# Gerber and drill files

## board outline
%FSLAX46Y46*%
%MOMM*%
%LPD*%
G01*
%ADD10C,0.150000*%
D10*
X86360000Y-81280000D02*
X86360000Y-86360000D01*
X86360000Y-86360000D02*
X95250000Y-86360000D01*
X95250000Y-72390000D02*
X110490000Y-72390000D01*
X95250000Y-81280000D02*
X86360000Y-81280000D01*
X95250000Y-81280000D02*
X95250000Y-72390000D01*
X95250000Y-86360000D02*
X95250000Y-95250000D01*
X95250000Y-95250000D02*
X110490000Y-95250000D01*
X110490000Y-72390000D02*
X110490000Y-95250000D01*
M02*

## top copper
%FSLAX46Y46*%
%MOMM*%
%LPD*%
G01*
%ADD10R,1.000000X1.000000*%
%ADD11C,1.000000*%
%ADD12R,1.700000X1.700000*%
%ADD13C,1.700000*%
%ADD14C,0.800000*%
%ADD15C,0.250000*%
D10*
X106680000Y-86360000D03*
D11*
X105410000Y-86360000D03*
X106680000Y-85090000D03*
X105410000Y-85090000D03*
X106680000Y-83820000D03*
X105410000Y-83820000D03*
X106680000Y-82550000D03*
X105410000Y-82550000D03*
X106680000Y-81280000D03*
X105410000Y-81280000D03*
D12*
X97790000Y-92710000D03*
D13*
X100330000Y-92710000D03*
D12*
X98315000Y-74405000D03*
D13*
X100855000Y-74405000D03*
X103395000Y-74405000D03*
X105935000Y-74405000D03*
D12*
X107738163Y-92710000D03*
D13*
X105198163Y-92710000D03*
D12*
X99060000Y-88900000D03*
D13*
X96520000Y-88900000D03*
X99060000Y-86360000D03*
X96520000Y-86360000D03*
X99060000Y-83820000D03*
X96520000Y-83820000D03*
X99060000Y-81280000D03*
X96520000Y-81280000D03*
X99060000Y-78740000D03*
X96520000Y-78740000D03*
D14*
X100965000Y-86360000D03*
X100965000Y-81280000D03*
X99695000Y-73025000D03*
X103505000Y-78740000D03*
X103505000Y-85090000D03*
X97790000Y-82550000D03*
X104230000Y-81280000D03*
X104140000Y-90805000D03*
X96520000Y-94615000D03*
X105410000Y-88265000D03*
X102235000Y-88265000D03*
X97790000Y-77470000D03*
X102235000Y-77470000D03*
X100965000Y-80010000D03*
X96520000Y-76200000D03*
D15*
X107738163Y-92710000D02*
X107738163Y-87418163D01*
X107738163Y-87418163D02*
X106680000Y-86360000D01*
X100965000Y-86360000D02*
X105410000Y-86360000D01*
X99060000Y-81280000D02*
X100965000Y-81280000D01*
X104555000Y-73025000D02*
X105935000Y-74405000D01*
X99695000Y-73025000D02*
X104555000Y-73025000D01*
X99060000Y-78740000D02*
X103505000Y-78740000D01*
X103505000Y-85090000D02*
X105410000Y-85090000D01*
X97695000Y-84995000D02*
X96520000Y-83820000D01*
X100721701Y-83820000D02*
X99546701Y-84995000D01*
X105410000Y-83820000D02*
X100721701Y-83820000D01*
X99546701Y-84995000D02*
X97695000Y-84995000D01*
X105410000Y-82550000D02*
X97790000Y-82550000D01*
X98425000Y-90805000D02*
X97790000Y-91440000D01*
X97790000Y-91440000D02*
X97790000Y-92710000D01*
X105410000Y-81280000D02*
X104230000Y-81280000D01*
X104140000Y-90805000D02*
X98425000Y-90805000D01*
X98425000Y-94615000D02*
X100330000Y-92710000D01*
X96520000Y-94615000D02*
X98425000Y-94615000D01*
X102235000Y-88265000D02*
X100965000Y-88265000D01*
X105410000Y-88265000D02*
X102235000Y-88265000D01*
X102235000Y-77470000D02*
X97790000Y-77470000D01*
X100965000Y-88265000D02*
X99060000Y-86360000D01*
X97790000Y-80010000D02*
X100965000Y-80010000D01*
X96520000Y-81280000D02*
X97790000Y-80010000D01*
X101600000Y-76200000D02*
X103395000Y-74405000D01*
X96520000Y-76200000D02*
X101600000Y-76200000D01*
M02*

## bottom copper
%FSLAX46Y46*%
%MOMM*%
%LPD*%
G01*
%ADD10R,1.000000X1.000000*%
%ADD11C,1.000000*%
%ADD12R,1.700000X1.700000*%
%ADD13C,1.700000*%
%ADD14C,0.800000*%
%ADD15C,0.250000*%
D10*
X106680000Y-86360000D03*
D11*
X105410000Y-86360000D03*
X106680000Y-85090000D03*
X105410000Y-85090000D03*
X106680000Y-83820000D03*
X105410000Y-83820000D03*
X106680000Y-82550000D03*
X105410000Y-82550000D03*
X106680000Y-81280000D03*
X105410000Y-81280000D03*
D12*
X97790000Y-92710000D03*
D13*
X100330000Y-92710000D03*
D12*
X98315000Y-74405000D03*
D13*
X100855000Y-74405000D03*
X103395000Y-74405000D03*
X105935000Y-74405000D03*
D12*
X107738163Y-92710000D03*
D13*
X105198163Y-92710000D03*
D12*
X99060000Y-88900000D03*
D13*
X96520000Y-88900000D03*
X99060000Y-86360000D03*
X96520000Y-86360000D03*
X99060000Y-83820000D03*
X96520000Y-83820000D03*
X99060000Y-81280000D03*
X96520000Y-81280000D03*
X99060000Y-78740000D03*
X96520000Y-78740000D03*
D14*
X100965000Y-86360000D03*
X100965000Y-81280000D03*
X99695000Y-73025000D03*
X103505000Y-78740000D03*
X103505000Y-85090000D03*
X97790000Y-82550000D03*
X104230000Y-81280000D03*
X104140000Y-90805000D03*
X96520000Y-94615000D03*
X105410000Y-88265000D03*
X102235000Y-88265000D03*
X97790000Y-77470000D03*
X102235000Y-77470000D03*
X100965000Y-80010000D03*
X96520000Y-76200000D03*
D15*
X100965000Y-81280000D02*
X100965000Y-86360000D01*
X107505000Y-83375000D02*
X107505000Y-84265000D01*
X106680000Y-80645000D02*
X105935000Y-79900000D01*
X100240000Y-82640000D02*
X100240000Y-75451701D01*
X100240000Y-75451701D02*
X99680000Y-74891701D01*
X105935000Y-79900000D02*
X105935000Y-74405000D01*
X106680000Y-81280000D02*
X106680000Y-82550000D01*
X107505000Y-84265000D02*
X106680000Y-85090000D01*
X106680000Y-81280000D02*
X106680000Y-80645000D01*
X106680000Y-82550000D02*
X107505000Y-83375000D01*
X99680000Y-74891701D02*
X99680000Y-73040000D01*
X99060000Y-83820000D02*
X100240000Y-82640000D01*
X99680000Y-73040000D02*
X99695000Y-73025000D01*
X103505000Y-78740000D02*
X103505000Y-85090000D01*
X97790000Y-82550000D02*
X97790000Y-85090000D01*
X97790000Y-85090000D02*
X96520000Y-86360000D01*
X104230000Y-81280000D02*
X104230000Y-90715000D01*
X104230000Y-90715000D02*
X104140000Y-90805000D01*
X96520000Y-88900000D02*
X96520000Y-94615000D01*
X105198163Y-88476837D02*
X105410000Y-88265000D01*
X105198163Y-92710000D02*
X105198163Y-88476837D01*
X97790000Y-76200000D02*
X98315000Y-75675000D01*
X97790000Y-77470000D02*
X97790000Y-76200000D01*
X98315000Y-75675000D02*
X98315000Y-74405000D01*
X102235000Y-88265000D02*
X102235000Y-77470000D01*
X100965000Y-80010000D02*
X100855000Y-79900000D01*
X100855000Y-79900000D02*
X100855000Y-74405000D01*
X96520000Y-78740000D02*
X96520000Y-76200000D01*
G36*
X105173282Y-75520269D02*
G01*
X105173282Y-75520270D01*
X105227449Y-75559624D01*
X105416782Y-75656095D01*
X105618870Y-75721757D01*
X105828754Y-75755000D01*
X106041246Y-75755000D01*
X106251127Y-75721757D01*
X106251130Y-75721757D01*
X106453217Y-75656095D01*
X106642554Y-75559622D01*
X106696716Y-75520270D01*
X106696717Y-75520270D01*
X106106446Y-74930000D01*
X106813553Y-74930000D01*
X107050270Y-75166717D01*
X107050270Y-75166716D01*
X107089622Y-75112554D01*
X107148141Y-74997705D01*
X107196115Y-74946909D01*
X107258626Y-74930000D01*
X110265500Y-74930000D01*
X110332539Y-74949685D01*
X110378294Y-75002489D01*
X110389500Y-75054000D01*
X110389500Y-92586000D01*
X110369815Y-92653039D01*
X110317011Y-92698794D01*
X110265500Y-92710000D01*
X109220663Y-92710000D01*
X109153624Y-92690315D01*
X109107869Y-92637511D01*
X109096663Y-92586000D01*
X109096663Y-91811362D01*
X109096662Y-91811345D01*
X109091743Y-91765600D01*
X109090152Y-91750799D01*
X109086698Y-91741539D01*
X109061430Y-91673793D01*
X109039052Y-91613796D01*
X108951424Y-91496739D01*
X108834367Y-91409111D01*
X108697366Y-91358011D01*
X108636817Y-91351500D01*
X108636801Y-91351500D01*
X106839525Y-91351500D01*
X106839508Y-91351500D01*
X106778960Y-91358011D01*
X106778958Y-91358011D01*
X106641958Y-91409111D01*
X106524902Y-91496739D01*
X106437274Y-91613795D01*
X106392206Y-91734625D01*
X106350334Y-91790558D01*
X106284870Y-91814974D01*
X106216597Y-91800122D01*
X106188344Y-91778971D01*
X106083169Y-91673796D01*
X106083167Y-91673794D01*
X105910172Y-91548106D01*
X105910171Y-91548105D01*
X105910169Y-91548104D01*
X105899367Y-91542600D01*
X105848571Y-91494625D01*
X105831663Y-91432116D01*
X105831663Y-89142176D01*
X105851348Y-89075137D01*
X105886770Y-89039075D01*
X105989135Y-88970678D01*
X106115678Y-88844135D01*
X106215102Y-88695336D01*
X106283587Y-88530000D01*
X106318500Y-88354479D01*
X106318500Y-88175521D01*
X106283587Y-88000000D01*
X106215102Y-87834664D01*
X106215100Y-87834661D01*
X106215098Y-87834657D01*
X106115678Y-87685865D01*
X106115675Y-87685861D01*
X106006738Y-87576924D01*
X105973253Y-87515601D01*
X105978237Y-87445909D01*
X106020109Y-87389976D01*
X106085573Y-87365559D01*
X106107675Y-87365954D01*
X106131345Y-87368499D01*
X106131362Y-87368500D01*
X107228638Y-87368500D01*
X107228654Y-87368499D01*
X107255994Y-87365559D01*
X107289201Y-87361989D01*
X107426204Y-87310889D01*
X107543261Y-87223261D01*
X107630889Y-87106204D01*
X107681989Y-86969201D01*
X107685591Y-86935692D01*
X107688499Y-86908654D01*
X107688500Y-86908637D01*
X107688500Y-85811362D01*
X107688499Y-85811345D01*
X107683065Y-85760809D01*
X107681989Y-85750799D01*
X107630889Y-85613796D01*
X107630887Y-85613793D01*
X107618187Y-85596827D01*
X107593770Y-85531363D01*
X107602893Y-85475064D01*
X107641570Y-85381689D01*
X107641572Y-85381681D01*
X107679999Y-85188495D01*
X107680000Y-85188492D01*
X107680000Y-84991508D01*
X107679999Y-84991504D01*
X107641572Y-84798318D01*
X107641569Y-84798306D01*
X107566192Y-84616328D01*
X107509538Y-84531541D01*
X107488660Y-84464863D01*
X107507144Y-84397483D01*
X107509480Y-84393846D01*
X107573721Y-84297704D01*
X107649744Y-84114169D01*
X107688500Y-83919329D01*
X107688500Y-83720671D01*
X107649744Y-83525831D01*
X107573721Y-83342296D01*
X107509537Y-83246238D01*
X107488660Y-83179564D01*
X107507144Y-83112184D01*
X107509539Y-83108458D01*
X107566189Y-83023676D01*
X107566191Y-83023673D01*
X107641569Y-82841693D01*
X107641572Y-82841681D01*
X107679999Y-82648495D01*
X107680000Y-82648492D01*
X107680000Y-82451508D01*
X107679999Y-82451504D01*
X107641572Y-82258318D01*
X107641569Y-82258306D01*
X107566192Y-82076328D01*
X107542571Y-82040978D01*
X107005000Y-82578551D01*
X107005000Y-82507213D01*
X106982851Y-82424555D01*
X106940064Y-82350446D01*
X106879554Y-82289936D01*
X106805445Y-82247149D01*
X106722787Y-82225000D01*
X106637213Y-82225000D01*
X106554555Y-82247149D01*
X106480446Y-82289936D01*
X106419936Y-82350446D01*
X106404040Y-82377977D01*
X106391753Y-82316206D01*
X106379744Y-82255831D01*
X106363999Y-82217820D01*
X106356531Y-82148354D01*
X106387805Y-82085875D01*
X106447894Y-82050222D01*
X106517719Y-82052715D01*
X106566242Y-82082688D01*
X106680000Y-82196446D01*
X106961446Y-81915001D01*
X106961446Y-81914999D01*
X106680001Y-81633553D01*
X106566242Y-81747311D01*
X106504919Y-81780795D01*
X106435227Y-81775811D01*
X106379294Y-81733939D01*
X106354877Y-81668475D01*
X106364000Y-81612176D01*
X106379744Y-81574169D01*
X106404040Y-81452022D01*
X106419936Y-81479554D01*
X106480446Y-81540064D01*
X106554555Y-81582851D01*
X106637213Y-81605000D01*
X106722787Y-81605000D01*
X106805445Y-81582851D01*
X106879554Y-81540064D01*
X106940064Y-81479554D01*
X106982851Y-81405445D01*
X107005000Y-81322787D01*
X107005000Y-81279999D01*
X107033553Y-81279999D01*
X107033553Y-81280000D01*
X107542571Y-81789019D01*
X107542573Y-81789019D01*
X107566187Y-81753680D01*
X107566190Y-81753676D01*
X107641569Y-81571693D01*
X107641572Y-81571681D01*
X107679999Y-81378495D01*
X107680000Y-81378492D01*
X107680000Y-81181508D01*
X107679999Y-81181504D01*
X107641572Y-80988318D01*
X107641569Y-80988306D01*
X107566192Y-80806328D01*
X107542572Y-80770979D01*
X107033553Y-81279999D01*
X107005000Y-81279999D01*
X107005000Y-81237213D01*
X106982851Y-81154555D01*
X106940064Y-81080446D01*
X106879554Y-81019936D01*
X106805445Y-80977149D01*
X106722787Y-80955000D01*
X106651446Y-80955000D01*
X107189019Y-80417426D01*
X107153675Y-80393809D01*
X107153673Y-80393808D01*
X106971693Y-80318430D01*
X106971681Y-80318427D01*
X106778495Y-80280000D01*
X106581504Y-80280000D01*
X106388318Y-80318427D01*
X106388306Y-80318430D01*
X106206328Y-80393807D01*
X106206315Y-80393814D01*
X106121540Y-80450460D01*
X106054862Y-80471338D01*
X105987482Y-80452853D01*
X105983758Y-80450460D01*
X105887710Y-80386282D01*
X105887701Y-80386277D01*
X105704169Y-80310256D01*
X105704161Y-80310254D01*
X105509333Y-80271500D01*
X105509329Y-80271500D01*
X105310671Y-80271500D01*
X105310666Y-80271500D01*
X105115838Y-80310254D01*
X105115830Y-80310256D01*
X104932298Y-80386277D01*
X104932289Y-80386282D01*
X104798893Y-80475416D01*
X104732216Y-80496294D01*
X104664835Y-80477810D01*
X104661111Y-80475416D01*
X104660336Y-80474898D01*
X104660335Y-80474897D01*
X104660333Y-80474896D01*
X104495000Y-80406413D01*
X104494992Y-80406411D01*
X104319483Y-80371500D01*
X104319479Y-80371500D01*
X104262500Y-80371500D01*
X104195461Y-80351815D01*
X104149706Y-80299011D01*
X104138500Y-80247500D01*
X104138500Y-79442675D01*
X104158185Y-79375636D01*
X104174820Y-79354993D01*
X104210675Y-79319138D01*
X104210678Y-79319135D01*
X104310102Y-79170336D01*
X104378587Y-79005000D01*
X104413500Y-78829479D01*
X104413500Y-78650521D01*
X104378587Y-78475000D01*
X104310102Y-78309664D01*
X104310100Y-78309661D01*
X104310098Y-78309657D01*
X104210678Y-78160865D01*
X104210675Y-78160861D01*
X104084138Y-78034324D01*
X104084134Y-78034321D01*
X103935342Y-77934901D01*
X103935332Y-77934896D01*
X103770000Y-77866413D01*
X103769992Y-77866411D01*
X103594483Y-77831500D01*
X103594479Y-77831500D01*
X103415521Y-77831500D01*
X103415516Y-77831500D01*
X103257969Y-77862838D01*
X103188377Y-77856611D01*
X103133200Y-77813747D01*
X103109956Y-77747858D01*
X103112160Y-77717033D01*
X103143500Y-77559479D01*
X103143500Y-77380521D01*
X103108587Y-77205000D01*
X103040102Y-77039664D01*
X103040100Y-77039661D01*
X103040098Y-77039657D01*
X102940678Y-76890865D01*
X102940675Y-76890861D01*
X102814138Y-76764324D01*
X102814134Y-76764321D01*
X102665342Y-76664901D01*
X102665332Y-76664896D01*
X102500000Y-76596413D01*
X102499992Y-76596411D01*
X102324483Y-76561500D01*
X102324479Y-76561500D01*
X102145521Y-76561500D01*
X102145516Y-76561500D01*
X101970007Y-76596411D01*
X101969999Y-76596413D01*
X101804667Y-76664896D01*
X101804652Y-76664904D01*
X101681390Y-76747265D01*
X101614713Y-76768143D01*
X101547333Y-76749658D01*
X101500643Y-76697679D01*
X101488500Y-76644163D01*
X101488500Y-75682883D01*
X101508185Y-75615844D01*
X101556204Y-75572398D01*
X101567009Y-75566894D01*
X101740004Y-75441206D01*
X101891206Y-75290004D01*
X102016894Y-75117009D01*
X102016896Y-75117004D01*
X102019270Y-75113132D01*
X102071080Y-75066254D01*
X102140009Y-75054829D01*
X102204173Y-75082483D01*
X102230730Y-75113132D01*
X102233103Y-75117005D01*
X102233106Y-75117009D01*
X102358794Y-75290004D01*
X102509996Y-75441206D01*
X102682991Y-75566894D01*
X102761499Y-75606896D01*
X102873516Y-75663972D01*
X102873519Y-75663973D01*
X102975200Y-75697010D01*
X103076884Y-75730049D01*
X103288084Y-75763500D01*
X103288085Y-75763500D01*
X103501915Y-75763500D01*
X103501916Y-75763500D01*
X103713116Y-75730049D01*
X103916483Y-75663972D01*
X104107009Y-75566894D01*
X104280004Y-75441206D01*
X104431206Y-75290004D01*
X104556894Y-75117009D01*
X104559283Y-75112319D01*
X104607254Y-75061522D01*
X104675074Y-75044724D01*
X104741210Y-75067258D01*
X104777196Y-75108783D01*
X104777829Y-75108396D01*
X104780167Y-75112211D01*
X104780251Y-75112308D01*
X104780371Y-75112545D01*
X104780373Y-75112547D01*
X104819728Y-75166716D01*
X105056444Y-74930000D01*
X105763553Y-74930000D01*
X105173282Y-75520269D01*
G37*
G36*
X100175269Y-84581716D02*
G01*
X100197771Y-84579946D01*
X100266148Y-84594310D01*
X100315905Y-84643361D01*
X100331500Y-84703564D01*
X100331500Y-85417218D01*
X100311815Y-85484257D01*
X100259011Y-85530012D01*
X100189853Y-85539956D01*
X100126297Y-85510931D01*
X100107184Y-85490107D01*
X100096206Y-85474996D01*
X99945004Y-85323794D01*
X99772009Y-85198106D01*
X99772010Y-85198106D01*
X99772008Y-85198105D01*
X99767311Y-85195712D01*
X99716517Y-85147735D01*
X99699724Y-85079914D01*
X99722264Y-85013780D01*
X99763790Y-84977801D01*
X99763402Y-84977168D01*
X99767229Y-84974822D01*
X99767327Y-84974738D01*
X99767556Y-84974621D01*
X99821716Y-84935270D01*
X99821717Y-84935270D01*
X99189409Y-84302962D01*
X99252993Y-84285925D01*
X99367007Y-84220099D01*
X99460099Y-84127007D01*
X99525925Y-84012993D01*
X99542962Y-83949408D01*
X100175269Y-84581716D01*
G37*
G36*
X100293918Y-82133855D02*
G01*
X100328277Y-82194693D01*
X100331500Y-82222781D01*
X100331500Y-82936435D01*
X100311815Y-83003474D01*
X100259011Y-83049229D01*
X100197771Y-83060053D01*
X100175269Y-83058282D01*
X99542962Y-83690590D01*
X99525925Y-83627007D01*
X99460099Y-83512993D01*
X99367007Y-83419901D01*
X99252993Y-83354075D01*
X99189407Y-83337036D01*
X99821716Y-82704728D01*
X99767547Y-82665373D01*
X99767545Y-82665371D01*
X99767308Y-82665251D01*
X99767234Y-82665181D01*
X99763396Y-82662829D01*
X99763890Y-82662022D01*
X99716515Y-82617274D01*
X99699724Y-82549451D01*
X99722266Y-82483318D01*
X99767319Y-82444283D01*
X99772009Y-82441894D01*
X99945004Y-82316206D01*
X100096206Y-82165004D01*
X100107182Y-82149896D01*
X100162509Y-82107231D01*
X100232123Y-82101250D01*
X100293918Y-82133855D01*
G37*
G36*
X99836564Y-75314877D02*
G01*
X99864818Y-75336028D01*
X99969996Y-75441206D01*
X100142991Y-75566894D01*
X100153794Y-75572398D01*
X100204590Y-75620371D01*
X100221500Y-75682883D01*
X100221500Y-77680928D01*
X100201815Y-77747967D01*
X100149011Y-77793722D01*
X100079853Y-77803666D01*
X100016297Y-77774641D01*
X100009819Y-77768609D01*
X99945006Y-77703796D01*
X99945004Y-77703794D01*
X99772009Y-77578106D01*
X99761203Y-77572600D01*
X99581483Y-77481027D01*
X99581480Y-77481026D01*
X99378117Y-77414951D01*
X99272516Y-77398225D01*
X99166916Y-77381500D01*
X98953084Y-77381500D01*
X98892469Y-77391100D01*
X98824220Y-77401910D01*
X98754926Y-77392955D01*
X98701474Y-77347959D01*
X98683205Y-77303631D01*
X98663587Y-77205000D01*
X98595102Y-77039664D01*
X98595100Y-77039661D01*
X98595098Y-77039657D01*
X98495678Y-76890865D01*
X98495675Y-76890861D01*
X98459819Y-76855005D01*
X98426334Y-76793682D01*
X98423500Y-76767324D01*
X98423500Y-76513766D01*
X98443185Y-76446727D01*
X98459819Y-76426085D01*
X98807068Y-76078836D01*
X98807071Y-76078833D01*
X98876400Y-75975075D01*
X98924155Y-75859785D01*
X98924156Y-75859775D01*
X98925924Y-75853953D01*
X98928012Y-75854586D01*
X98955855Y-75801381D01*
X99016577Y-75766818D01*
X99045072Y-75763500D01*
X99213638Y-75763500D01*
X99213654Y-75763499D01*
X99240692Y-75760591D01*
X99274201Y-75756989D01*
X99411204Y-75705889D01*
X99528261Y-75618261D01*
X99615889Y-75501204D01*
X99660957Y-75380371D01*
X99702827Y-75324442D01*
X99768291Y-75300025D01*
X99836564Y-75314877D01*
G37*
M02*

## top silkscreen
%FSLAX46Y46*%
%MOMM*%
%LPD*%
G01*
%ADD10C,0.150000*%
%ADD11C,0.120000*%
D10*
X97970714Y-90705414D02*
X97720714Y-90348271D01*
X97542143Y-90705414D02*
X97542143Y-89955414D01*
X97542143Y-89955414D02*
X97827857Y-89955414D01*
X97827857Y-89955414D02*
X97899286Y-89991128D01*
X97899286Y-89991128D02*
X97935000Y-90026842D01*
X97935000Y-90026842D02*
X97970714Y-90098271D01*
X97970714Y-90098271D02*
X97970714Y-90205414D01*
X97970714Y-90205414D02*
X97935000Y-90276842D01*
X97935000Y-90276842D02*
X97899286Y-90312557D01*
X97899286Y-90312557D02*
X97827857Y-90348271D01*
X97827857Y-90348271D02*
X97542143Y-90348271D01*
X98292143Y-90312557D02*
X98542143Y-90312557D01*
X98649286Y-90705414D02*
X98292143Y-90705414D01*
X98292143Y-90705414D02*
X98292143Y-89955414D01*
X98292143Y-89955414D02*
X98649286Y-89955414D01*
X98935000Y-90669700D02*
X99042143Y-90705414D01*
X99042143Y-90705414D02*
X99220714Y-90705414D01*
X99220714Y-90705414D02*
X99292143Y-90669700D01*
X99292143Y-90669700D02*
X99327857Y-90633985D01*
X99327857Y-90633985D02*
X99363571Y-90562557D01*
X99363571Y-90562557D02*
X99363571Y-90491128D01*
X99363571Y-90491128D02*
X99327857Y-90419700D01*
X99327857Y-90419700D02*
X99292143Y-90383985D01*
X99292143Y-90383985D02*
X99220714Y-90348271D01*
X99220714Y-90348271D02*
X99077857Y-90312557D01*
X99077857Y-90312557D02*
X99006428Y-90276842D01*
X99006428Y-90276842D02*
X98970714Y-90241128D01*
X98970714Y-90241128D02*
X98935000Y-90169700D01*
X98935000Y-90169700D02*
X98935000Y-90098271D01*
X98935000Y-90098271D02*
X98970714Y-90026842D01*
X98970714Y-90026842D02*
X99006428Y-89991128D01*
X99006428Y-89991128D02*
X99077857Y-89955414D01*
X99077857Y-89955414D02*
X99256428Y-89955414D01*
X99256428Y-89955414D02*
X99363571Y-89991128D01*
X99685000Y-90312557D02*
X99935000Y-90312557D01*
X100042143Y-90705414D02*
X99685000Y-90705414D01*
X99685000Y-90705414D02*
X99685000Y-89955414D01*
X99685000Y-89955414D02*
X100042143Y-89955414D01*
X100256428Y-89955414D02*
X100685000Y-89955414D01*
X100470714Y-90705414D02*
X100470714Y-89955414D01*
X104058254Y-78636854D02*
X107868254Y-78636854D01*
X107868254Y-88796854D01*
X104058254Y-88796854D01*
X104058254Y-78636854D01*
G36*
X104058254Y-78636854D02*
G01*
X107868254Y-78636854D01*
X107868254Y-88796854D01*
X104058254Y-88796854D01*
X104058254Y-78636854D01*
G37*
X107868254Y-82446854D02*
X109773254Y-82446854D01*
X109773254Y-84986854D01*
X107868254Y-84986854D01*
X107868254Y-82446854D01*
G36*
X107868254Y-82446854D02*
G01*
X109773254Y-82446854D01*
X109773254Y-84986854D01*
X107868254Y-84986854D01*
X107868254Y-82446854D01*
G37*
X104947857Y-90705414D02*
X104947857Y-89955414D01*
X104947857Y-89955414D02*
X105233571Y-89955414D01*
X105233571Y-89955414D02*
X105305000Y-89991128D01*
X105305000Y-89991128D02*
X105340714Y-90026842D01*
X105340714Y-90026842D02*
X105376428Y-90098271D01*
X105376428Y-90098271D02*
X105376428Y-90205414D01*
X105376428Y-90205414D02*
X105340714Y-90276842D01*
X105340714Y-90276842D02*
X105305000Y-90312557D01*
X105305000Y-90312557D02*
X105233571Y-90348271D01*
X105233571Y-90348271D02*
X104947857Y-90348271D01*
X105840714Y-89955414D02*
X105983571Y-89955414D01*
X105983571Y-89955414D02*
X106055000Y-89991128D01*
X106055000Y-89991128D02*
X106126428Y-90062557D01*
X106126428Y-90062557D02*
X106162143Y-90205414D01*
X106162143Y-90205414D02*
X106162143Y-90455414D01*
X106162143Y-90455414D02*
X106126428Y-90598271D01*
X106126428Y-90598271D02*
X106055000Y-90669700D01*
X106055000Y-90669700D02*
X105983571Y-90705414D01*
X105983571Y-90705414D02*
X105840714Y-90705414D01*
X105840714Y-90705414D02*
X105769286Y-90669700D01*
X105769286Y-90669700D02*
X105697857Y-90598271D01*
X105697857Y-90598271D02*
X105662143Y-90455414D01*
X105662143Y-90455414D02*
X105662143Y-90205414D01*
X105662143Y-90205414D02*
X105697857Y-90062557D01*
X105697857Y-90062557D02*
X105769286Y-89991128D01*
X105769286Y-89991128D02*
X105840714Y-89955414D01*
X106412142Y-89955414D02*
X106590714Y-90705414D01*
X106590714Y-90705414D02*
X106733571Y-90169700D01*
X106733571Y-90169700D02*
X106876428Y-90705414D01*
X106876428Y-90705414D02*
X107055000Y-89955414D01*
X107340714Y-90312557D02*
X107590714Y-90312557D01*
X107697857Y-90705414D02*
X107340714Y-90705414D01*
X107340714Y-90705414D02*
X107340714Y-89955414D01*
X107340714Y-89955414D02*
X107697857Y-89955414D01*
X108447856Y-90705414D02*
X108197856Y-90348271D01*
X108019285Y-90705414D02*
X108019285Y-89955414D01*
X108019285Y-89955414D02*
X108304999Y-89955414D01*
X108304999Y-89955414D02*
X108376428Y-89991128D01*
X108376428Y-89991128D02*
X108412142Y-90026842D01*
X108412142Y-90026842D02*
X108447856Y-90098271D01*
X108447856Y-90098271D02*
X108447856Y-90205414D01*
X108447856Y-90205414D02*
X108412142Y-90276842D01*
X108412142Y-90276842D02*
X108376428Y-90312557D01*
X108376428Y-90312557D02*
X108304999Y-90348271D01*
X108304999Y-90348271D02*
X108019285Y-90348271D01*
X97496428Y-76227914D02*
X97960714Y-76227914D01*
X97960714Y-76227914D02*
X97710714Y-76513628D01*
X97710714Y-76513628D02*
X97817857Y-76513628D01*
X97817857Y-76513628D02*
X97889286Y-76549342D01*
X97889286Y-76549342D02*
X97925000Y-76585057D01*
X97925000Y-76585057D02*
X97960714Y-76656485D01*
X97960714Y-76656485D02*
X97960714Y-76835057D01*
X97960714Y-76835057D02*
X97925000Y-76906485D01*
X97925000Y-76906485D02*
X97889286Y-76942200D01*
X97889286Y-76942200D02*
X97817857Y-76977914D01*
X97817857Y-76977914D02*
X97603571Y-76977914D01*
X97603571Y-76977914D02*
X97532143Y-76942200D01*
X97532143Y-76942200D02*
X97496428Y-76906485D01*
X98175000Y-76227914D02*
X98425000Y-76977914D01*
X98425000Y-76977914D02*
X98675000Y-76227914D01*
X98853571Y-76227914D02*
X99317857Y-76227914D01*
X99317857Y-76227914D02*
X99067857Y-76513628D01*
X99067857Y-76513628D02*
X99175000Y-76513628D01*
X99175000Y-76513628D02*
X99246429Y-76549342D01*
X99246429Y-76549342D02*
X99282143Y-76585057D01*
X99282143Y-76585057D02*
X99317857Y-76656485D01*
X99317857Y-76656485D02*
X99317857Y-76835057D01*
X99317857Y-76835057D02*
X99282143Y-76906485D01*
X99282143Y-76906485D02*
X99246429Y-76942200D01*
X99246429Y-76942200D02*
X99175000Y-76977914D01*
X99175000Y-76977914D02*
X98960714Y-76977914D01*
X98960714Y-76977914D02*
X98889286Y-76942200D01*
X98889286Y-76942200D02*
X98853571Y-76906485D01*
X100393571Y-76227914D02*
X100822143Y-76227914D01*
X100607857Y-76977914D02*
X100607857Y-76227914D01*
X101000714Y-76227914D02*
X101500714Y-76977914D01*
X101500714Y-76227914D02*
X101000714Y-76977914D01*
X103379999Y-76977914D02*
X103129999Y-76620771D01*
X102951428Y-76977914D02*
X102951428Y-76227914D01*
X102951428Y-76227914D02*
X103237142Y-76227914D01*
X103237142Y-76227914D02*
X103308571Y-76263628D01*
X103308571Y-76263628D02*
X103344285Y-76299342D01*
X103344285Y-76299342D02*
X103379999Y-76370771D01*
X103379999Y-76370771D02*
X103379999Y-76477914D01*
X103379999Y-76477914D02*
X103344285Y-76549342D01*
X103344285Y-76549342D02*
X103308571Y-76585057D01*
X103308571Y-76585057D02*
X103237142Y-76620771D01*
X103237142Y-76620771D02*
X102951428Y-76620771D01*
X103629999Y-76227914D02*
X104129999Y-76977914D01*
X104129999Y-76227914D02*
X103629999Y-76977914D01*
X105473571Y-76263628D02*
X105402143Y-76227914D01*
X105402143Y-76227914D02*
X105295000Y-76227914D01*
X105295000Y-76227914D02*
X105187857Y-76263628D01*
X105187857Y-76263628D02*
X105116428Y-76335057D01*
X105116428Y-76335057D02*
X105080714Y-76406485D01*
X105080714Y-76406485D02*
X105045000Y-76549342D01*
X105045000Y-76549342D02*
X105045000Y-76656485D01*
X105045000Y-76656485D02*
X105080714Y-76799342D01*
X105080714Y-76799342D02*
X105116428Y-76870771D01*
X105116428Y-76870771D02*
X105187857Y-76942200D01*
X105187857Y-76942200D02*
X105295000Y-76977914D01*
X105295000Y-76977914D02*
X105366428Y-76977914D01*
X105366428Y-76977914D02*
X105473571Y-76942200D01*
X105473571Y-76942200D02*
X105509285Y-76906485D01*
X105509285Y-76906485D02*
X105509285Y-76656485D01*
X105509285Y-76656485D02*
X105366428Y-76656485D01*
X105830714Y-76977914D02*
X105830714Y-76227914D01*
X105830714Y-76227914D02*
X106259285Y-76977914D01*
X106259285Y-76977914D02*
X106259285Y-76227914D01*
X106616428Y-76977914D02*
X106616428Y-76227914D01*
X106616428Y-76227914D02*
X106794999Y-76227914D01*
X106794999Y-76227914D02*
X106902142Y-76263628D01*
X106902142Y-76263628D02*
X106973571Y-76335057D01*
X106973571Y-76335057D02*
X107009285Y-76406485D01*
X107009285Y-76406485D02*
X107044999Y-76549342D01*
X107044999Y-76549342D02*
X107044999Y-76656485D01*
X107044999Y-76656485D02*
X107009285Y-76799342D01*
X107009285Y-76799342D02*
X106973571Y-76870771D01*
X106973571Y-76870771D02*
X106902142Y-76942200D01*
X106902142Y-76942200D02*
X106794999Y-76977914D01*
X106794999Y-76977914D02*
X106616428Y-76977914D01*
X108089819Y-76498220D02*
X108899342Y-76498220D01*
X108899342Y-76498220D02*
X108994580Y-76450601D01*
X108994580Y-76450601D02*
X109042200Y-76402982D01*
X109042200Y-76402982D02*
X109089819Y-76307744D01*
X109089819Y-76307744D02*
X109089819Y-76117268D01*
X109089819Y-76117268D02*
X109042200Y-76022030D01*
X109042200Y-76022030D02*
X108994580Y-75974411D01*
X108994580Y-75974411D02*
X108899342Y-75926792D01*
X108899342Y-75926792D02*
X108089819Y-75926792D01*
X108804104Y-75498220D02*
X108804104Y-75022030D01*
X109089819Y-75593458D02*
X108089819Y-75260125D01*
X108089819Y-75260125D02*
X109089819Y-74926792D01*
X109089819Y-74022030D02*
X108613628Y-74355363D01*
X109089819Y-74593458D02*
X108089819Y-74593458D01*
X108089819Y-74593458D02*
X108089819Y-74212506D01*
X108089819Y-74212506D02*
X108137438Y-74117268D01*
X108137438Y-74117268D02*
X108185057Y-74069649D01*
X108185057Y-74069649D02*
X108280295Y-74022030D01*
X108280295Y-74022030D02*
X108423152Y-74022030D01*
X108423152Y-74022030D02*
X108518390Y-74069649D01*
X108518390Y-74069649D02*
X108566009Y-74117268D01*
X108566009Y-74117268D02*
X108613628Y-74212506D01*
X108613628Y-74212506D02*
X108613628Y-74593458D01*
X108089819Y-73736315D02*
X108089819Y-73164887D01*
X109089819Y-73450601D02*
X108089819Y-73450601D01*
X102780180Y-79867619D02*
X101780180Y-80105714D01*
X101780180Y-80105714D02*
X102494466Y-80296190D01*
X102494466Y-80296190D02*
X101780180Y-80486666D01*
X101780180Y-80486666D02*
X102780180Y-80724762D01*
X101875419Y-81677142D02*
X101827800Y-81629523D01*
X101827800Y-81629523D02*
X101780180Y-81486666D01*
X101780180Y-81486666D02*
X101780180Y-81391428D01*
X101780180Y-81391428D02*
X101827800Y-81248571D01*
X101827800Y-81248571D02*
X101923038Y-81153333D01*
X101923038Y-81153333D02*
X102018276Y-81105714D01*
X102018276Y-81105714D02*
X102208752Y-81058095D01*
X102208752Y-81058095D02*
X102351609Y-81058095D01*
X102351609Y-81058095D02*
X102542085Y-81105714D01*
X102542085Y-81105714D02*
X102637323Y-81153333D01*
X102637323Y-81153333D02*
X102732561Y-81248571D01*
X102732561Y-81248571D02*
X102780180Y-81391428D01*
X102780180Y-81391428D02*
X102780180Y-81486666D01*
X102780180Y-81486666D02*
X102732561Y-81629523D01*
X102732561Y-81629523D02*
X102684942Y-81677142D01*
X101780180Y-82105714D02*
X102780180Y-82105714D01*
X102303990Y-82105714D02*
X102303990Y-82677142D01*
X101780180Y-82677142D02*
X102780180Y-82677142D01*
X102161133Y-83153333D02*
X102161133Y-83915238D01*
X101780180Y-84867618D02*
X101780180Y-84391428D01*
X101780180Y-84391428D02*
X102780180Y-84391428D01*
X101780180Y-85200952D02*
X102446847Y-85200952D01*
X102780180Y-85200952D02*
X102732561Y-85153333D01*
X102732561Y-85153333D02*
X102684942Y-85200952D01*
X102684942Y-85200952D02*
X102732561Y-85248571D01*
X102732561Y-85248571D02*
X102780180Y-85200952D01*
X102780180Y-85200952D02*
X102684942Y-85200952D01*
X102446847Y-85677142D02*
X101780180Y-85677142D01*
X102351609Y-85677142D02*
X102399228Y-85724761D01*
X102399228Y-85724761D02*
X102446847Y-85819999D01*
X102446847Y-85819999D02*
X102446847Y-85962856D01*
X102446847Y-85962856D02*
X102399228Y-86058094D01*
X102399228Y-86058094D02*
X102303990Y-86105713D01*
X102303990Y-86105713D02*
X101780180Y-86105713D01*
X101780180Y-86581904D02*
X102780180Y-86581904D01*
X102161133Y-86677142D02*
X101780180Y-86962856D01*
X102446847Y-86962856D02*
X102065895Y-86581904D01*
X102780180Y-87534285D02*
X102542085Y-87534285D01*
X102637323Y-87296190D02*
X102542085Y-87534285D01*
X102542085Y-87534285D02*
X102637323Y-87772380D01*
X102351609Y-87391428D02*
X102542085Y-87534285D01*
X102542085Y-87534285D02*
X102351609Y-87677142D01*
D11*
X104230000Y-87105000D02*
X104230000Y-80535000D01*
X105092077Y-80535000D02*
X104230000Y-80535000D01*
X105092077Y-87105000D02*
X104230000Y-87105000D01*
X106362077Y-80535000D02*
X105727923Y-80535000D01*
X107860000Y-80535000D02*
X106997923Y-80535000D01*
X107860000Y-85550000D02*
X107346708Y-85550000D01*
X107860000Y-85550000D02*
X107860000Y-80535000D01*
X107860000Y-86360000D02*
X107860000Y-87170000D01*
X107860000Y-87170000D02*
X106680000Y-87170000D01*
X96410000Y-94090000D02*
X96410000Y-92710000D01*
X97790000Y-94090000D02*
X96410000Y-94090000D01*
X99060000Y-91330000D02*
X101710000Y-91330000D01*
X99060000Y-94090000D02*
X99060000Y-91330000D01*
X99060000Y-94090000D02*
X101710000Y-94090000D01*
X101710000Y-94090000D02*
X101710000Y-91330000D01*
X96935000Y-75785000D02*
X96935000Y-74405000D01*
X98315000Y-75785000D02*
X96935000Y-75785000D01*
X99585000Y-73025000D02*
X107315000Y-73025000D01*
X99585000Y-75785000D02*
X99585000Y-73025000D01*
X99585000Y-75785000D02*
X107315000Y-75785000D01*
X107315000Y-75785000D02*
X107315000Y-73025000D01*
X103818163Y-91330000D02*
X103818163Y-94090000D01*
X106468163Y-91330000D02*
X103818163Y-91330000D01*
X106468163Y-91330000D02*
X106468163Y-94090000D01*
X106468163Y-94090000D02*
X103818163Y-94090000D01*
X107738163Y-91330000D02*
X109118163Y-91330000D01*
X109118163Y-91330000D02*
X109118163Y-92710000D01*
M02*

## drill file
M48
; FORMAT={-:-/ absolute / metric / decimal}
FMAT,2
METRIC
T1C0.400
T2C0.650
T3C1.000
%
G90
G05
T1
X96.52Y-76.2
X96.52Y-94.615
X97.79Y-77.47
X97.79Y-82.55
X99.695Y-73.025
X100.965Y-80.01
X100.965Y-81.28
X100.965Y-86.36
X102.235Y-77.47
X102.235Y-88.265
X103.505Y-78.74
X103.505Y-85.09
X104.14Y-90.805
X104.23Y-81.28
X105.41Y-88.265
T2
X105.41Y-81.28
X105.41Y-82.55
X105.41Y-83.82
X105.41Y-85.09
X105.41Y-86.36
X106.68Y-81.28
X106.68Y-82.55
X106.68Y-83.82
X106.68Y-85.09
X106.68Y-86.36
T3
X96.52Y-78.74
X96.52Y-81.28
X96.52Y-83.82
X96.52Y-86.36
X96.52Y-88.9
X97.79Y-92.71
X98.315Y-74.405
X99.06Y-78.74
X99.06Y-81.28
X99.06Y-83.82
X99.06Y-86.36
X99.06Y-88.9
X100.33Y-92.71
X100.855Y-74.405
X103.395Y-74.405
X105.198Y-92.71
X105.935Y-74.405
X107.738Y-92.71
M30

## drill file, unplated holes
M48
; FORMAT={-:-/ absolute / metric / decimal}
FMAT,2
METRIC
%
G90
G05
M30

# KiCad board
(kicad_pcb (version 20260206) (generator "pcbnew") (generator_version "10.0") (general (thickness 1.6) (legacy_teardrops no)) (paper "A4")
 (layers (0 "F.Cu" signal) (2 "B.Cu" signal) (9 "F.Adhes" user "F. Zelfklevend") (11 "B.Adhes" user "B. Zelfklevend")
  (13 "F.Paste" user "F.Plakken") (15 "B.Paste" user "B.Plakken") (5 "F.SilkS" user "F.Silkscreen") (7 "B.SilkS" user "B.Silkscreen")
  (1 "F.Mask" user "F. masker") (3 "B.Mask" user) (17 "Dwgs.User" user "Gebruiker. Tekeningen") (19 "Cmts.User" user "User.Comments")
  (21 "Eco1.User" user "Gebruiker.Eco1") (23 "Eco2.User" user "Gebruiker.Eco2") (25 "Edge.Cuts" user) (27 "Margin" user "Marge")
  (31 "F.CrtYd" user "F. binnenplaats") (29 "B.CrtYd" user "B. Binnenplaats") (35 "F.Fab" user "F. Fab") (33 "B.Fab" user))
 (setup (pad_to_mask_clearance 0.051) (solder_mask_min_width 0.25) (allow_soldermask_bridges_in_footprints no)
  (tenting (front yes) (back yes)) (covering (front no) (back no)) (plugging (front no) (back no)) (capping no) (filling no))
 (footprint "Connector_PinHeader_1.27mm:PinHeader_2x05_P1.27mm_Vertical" (layer "F.Cu") (at 106.68 86.36 180)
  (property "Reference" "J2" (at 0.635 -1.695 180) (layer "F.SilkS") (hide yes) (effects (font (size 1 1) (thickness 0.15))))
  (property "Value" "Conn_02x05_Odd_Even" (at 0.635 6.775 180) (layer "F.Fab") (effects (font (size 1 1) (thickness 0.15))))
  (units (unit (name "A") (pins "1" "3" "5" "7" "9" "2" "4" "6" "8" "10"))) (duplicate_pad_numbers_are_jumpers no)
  (fp_line (start 2.45 -0.745) (end 2.45 5.825) (stroke (width 0.12) (type solid)) (layer "F.SilkS"))
  (fp_line (start 1.587923 5.825) (end 2.45 5.825) (stroke (width 0.12) (type solid)) (layer "F.SilkS"))
  (fp_line (start 1.587923 -0.745) (end 2.45 -0.745) (stroke (width 0.12) (type solid)) (layer "F.SilkS"))
  (fp_line (start 0.317923 5.825) (end 0.952077 5.825) (stroke (width 0.12) (type solid)) (layer "F.SilkS"))
  (fp_line (start -1.18 5.825) (end -0.317923 5.825) (stroke (width 0.12) (type solid)) (layer "F.SilkS"))
  (fp_line (start -1.18 0.81) (end -0.666708 0.81) (stroke (width 0.12) (type solid)) (layer "F.SilkS"))
  (fp_line (start -1.18 0.81) (end -1.18 5.825) (stroke (width 0.12) (type solid)) (layer "F.SilkS"))
  (fp_line (start -1.18 0) (end -1.18 -0.81) (stroke (width 0.12) (type solid)) (layer "F.SilkS"))
  (fp_line (start -1.18 -0.81) (end 0 -0.81) (stroke (width 0.12) (type solid)) (layer "F.SilkS"))
  (pad "1" thru_hole rect (at 0 0 180) (size 1 1) (drill 0.65) (layers "*.Cu" "*.Mask") (remove_unused_layers no) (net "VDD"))
  (pad "2" thru_hole circle (at 1.27 0 180) (size 1 1) (drill 0.65) (layers "*.Cu" "*.Mask") (remove_unused_layers no) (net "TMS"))
  (pad "3" thru_hole circle (at 0 1.27 180) (size 1 1) (drill 0.65) (layers "*.Cu" "*.Mask") (remove_unused_layers no) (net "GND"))
  (pad "4" thru_hole circle (at 1.27 1.27 180) (size 1 1) (drill 0.65) (layers "*.Cu" "*.Mask") (remove_unused_layers no) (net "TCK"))
  (pad "5" thru_hole circle (at 0 2.54 180) (size 1 1) (drill 0.65) (layers "*.Cu" "*.Mask") (remove_unused_layers no)
   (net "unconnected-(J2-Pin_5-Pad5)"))
  (pad "6" thru_hole circle (at 1.27 2.54 180) (size 1 1) (drill 0.65) (layers "*.Cu" "*.Mask") (remove_unused_layers no) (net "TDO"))
  (pad "7" thru_hole circle (at 0 3.81 180) (size 1 1) (drill 0.65) (layers "*.Cu" "*.Mask") (remove_unused_layers no) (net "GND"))
  (pad "8" thru_hole circle (at 1.27 3.81 180) (size 1 1) (drill 0.65) (layers "*.Cu" "*.Mask") (remove_unused_layers no) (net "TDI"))
  (pad "9" thru_hole circle (at 0 5.08 180) (size 1 1) (drill 0.65) (layers "*.Cu" "*.Mask") (remove_unused_layers no) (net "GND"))
  (pad "10" thru_hole circle (at 1.27 5.08 180) (size 1 1) (drill 0.65) (layers "*.Cu" "*.Mask") (remove_unused_layers no) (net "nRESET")))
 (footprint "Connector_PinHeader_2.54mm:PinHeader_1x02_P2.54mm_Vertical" (layer "F.Cu") (at 97.79 92.71 90)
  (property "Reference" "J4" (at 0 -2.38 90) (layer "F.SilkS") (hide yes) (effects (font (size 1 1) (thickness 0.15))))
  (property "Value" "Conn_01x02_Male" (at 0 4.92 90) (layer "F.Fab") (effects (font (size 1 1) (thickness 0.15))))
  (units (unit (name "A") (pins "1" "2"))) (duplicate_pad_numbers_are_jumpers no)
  (fp_line (start -1.38 -1.38) (end 0 -1.38) (stroke (width 0.12) (type solid)) (layer "F.SilkS"))
  (fp_line (start -1.38 0) (end -1.38 -1.38) (stroke (width 0.12) (type solid)) (layer "F.SilkS"))
  (fp_line (start 1.38 1.27) (end 1.38 3.92) (stroke (width 0.12) (type solid)) (layer "F.SilkS"))
  (fp_line (start -1.38 1.27) (end 1.38 1.27) (stroke (width 0.12) (type solid)) (layer "F.SilkS"))
  (fp_line (start -1.38 1.27) (end -1.38 3.92) (stroke (width 0.12) (type solid)) (layer "F.SilkS"))
  (fp_line (start -1.38 3.92) (end 1.38 3.92) (stroke (width 0.12) (type solid)) (layer "F.SilkS"))
  (pad "1" thru_hole rect (at 0 0 90) (size 1.7 1.7) (drill 1) (layers "*.Cu" "*.Mask") (remove_unused_layers no) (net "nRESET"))
  (pad "2" thru_hole circle (at 0 2.54 90) (size 1.7 1.7) (drill 1) (layers "*.Cu" "*.Mask") (remove_unused_layers no) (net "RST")))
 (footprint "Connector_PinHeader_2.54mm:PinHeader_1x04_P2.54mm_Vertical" (layer "F.Cu") (at 98.315 74.405 90)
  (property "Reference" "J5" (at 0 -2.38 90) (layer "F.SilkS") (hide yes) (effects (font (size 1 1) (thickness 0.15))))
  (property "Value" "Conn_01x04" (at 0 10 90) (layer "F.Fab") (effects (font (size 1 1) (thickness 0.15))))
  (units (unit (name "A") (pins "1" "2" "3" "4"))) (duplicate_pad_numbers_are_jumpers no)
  (fp_line (start -1.38 -1.38) (end 0 -1.38) (stroke (width 0.12) (type solid)) (layer "F.SilkS"))
  (fp_line (start -1.38 0) (end -1.38 -1.38) (stroke (width 0.12) (type solid)) (layer "F.SilkS"))
  (fp_line (start 1.38 1.27) (end 1.38 9) (stroke (width 0.12) (type solid)) (layer "F.SilkS"))
  (fp_line (start -1.38 1.27) (end 1.38 1.27) (stroke (width 0.12) (type solid)) (layer "F.SilkS"))
  (fp_line (start -1.38 1.27) (end -1.38 9) (stroke (width 0.12) (type solid)) (layer "F.SilkS"))
  (fp_line (start -1.38 9) (end 1.38 9) (stroke (width 0.12) (type solid)) (layer "F.SilkS"))
  (pad "1" thru_hole rect (at 0 0 90) (size 1.7 1.7) (drill 1) (layers "*.Cu" "*.Mask") (remove_unused_layers no) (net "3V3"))
  (pad "2" thru_hole circle (at 0 2.54 90) (size 1.7 1.7) (drill 1) (layers "*.Cu" "*.Mask") (remove_unused_layers no) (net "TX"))
  (pad "3" thru_hole circle (at 0 5.08 90) (size 1.7 1.7) (drill 1) (layers "*.Cu" "*.Mask") (remove_unused_layers no) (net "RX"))
  (pad "4" thru_hole circle (at 0 7.62 90) (size 1.7 1.7) (drill 1) (layers "*.Cu" "*.Mask") (remove_unused_layers no) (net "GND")))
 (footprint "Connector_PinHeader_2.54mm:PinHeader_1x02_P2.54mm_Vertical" (layer "F.Cu") (at 107.738163 92.71 -90)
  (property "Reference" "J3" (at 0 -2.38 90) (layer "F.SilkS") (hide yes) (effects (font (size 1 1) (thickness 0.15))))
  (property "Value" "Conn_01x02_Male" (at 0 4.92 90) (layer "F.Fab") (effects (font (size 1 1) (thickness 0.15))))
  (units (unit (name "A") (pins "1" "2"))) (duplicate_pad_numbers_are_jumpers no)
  (fp_line (start -1.38 3.92) (end 1.38 3.92) (stroke (width 0.12) (type solid)) (layer "F.SilkS"))
  (fp_line (start -1.38 1.27) (end -1.38 3.92) (stroke (width 0.12) (type solid)) (layer "F.SilkS"))
  (fp_line (start -1.38 1.27) (end 1.38 1.27) (stroke (width 0.12) (type solid)) (layer "F.SilkS"))
  (fp_line (start 1.38 1.27) (end 1.38 3.92) (stroke (width 0.12) (type solid)) (layer "F.SilkS"))
  (fp_line (start -1.38 0) (end -1.38 -1.38) (stroke (width 0.12) (type solid)) (layer "F.SilkS"))
  (fp_line (start -1.38 -1.38) (end 0 -1.38) (stroke (width 0.12) (type solid)) (layer "F.SilkS"))
  (pad "1" thru_hole rect (at 0 0 270) (size 1.7 1.7) (drill 1) (layers "*.Cu" "*.Mask") (remove_unused_layers no) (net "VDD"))
  (pad "2" thru_hole circle (at 0 2.54 270) (size 1.7 1.7) (drill 1) (layers "*.Cu" "*.Mask") (remove_unused_layers no) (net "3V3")))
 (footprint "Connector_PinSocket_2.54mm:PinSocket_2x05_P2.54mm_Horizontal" (layer "B.Cu") (at 99.06 88.9)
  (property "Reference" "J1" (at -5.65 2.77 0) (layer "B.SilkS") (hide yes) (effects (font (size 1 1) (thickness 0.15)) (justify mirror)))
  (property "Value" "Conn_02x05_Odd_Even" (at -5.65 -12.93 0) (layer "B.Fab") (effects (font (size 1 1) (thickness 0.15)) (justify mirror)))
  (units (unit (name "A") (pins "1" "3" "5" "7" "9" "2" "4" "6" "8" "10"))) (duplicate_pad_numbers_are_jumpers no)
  (pad "1" thru_hole rect (at 0 0) (size 1.7 1.7) (drill 1) (layers "*.Cu" "*.Mask") (remove_unused_layers no) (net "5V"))
  (pad "2" thru_hole circle (at -2.54 0) (size 1.7 1.7) (drill 1) (layers "*.Cu" "*.Mask") (remove_unused_layers no) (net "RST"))
  (pad "3" thru_hole circle (at 0 -2.54) (size 1.7 1.7) (drill 1) (layers "*.Cu" "*.Mask") (remove_unused_layers no) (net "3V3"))
  (pad "4" thru_hole circle (at -2.54 -2.54) (size 1.7 1.7) (drill 1) (layers "*.Cu" "*.Mask") (remove_unused_layers no) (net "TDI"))
  (pad "5" thru_hole circle (at 0 -5.08) (size 1.7 1.7) (drill 1) (layers "*.Cu" "*.Mask") (remove_unused_layers no) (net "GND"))
  (pad "6" thru_hole circle (at -2.54 -5.08) (size 1.7 1.7) (drill 1) (layers "*.Cu" "*.Mask") (remove_unused_layers no) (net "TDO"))
  (pad "7" thru_hole circle (at 0 -7.62) (size 1.7 1.7) (drill 1) (layers "*.Cu" "*.Mask") (remove_unused_layers no) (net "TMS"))
  (pad "8" thru_hole circle (at -2.54 -7.62) (size 1.7 1.7) (drill 1) (layers "*.Cu" "*.Mask") (remove_unused_layers no) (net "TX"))
  (pad "9" thru_hole circle (at 0 -10.16) (size 1.7 1.7) (drill 1) (layers "*.Cu" "*.Mask") (remove_unused_layers no) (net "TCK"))
  (pad "10" thru_hole circle (at -2.54 -10.16) (size 1.7 1.7) (drill 1) (layers "*.Cu" "*.Mask") (remove_unused_layers no) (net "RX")))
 (gr_rect (start 104.058254 78.636854) (end 107.868254 88.796854) (stroke (width 0.15) (type solid)) (fill yes) (layer "F.SilkS"))
 (gr_rect (start 107.868254 82.446854) (end 109.773254 84.986854) (stroke (width 0.15) (type solid)) (fill yes) (layer "F.SilkS"))
 (gr_line (start 86.36 81.28) (end 86.36 86.36) (stroke (width 0.15) (type default)) (layer "Edge.Cuts"))
 (gr_line (start 86.36 86.36) (end 95.25 86.36) (stroke (width 0.15) (type default)) (layer "Edge.Cuts"))
 (gr_line (start 95.25 72.39) (end 110.49 72.39) (stroke (width 0.15) (type default)) (layer "Edge.Cuts"))
 (gr_line (start 95.25 81.28) (end 86.36 81.28) (stroke (width 0.15) (type default)) (layer "Edge.Cuts"))
 (gr_line (start 95.25 81.28) (end 95.25 72.39) (stroke (width 0.15) (type default)) (layer "Edge.Cuts"))
 (gr_line (start 95.25 86.36) (end 95.25 95.25) (stroke (width 0.15) (type default)) (layer "Edge.Cuts"))
 (gr_line (start 95.25 95.25) (end 110.49 95.25) (stroke (width 0.15) (type default)) (layer "Edge.Cuts"))
 (gr_line (start 110.49 72.39) (end 110.49 95.25) (stroke (width 0.15) (type default)) (layer "Edge.Cuts"))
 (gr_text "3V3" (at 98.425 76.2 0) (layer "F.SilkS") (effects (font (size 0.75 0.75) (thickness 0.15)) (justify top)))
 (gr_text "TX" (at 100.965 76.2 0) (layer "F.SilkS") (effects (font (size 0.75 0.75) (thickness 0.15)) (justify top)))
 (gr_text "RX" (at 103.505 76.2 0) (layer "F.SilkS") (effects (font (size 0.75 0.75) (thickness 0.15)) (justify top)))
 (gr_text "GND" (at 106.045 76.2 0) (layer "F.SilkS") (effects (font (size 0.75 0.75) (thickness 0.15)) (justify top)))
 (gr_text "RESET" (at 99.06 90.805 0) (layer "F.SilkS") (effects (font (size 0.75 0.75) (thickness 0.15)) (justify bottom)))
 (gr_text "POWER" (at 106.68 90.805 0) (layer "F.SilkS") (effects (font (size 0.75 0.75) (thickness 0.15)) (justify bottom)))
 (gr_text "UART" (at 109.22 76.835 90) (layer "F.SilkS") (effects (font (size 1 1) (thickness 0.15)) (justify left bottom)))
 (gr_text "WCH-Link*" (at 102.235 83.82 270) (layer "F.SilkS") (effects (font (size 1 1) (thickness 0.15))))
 (segment (start 107.738163 92.71) (end 107.738163 87.418163) (width 0.25) (layer "F.Cu") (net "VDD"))
 (segment (start 107.738163 87.418163) (end 106.68 86.36) (width 0.25) (layer "F.Cu") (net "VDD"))
 (segment (start 100.965 86.36) (end 105.41 86.36) (width 0.25) (layer "F.Cu") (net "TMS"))
 (segment (start 99.06 81.28) (end 100.965 81.28) (width 0.25) (layer "F.Cu") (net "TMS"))
 (via (at 100.965 86.36) (size 0.8) (drill 0.4) (layers "F.Cu" "B.Cu") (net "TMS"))
 (via (at 100.965 81.28) (size 0.8) (drill 0.4) (layers "F.Cu" "B.Cu") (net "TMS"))
 (segment (start 100.965 81.28) (end 100.965 86.36) (width 0.25) (layer "B.Cu") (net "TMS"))
 (segment (start 104.555 73.025) (end 105.935 74.405) (width 0.25) (layer "F.Cu") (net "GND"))
 (segment (start 99.695 73.025) (end 104.555 73.025) (width 0.25) (layer "F.Cu") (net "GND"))
 (via (at 99.695 73.025) (size 0.8) (drill 0.4) (layers "F.Cu" "B.Cu") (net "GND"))
 (segment (start 107.505 83.375) (end 107.505 84.265) (width 0.25) (layer "B.Cu") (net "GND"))
 (segment (start 106.68 80.645) (end 105.935 79.9) (width 0.25) (layer "B.Cu") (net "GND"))
 (segment (start 100.24 82.64) (end 100.24 75.451701) (width 0.25) (layer "B.Cu") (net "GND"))
 (segment (start 100.24 75.451701) (end 99.68 74.891701) (width 0.25) (layer "B.Cu") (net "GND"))
 (segment (start 105.935 79.9) (end 105.935 74.405) (width 0.25) (layer "B.Cu") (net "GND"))
 (segment (start 106.68 81.28) (end 106.68 82.55) (width 0.25) (layer "B.Cu") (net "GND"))
 (segment (start 107.505 84.265) (end 106.68 85.09) (width 0.25) (layer "B.Cu") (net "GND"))
 (segment (start 106.68 81.28) (end 106.68 80.645) (width 0.25) (layer "B.Cu") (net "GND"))
 (segment (start 106.68 82.55) (end 107.505 83.375) (width 0.25) (layer "B.Cu") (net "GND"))
 (segment (start 99.68 74.891701) (end 99.68 73.04) (width 0.25) (layer "B.Cu") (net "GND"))
 (segment (start 99.06 83.82) (end 100.24 82.64) (width 0.25) (layer "B.Cu") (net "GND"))
 (segment (start 99.68 73.04) (end 99.695 73.025) (width 0.25) (layer "B.Cu") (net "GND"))
 (segment (start 99.06 78.74) (end 103.505 78.74) (width 0.25) (layer "F.Cu") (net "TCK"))
 (segment (start 103.505 85.09) (end 105.41 85.09) (width 0.25) (layer "F.Cu") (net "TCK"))
 (via (at 103.505 78.74) (size 0.8) (drill 0.4) (layers "F.Cu" "B.Cu") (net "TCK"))
 (via (at 103.505 85.09) (size 0.8) (drill 0.4) (layers "F.Cu" "B.Cu") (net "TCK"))
 (segment (start 103.505 78.74) (end 103.505 85.09) (width 0.25) (layer "B.Cu") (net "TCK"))
 (segment (start 97.695 84.995) (end 96.52 83.82) (width 0.25) (layer "F.Cu") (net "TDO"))
 (segment (start 100.721701 83.82) (end 99.546701 84.995) (width 0.25) (layer "F.Cu") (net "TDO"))
 (segment (start 105.41 83.82) (end 100.721701 83.82) (width 0.25) (layer "F.Cu") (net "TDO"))
 (segment (start 99.546701 84.995) (end 97.695 84.995) (width 0.25) (layer "F.Cu") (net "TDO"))
 (segment (start 105.41 82.55) (end 97.79 82.55) (width 0.25) (layer "F.Cu") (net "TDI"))
 (via (at 97.79 82.55) (size 0.8) (drill 0.4) (layers "F.Cu" "B.Cu") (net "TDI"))
 (segment (start 97.79 82.55) (end 97.79 85.09) (width 0.25) (layer "B.Cu") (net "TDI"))
 (segment (start 97.79 85.09) (end 96.52 86.36) (width 0.25) (layer "B.Cu") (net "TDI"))
 (segment (start 98.425 90.805) (end 97.79 91.44) (width 0.25) (layer "F.Cu") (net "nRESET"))
 (segment (start 97.79 91.44) (end 97.79 92.71) (width 0.25) (layer "F.Cu") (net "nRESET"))
 (segment (start 105.41 81.28) (end 104.23 81.28) (width 0.25) (layer "F.Cu") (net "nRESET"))
 (segment (start 104.14 90.805) (end 98.425 90.805) (width 0.25) (layer "F.Cu") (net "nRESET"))
 (via (at 104.23 81.28) (size 0.8) (drill 0.4) (layers "F.Cu" "B.Cu") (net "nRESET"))
 (via (at 104.14 90.805) (size 0.8) (drill 0.4) (layers "F.Cu" "B.Cu") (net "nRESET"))
 (segment (start 104.23 81.28) (end 104.23 90.715) (width 0.25) (layer "B.Cu") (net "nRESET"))
 (segment (start 104.23 90.715) (end 104.14 90.805) (width 0.25) (layer "B.Cu") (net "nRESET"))
 (segment (start 98.425 94.615) (end 100.33 92.71) (width 0.25) (layer "F.Cu") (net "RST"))
 (segment (start 96.52 94.615) (end 98.425 94.615) (width 0.25) (layer "F.Cu") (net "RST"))
 (via (at 96.52 94.615) (size 0.8) (drill 0.4) (layers "F.Cu" "B.Cu") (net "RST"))
 (segment (start 96.52 88.9) (end 96.52 94.615) (width 0.25) (layer "B.Cu") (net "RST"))
 (segment (start 102.235 88.265) (end 100.965 88.265) (width 0.25) (layer "F.Cu") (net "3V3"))
 (segment (start 105.41 88.265) (end 102.235 88.265) (width 0.25) (layer "F.Cu") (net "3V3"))
 (segment (start 102.235 77.47) (end 97.79 77.47) (width 0.25) (layer "F.Cu") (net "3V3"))
 (segment (start 100.965 88.265) (end 99.06 86.36) (width 0.25) (layer "F.Cu") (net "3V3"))
 (via (at 105.41 88.265) (size 0.8) (drill 0.4) (layers "F.Cu" "B.Cu") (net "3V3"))
 (via (at 102.235 88.265) (size 0.8) (drill 0.4) (layers "F.Cu" "B.Cu") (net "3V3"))
 (via (at 97.79 77.47) (size 0.8) (drill 0.4) (layers "F.Cu" "B.Cu") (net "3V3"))
 (via (at 102.235 77.47) (size 0.8) (drill 0.4) (layers "F.Cu" "B.Cu") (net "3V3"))
 (segment (start 105.198163 88.476837) (end 105.41 88.265) (width 0.25) (layer "B.Cu") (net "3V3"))
 (segment (start 105.198163 92.71) (end 105.198163 88.476837) (width 0.25) (layer "B.Cu") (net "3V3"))
 (segment (start 97.79 76.2) (end 98.315 75.675) (width 0.25) (layer "B.Cu") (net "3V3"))
 (segment (start 97.79 77.47) (end 97.79 76.2) (width 0.25) (layer "B.Cu") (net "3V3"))
 (segment (start 98.315 75.675) (end 98.315 74.405) (width 0.25) (layer "B.Cu") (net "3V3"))
 (segment (start 102.235 88.265) (end 102.235 77.47) (width 0.25) (layer "B.Cu") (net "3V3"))
 (segment (start 97.79 80.01) (end 100.965 80.01) (width 0.25) (layer "F.Cu") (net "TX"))
 (segment (start 96.52 81.28) (end 97.79 80.01) (width 0.25) (layer "F.Cu") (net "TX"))
 (via (at 100.965 80.01) (size 0.8) (drill 0.4) (layers "F.Cu" "B.Cu") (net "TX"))
 (segment (start 100.965 80.01) (end 100.855 79.9) (width 0.25) (layer "B.Cu") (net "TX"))
 (segment (start 100.855 79.9) (end 100.855 74.405) (width 0.25) (layer "B.Cu") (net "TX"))
 (segment (start 101.6 76.2) (end 103.395 74.405) (width 0.25) (layer "F.Cu") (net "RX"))
 (segment (start 96.52 76.2) (end 101.6 76.2) (width 0.25) (layer "F.Cu") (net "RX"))
 (via (at 96.52 76.2) (size 0.8) (drill 0.4) (layers "F.Cu" "B.Cu") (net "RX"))
 (segment (start 96.52 78.74) (end 96.52 76.2) (width 0.25) (layer "B.Cu") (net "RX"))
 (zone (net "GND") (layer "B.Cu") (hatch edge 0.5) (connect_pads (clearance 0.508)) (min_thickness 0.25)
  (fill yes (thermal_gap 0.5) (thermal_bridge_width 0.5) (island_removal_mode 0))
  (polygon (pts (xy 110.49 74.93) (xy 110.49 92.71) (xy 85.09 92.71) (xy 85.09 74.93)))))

